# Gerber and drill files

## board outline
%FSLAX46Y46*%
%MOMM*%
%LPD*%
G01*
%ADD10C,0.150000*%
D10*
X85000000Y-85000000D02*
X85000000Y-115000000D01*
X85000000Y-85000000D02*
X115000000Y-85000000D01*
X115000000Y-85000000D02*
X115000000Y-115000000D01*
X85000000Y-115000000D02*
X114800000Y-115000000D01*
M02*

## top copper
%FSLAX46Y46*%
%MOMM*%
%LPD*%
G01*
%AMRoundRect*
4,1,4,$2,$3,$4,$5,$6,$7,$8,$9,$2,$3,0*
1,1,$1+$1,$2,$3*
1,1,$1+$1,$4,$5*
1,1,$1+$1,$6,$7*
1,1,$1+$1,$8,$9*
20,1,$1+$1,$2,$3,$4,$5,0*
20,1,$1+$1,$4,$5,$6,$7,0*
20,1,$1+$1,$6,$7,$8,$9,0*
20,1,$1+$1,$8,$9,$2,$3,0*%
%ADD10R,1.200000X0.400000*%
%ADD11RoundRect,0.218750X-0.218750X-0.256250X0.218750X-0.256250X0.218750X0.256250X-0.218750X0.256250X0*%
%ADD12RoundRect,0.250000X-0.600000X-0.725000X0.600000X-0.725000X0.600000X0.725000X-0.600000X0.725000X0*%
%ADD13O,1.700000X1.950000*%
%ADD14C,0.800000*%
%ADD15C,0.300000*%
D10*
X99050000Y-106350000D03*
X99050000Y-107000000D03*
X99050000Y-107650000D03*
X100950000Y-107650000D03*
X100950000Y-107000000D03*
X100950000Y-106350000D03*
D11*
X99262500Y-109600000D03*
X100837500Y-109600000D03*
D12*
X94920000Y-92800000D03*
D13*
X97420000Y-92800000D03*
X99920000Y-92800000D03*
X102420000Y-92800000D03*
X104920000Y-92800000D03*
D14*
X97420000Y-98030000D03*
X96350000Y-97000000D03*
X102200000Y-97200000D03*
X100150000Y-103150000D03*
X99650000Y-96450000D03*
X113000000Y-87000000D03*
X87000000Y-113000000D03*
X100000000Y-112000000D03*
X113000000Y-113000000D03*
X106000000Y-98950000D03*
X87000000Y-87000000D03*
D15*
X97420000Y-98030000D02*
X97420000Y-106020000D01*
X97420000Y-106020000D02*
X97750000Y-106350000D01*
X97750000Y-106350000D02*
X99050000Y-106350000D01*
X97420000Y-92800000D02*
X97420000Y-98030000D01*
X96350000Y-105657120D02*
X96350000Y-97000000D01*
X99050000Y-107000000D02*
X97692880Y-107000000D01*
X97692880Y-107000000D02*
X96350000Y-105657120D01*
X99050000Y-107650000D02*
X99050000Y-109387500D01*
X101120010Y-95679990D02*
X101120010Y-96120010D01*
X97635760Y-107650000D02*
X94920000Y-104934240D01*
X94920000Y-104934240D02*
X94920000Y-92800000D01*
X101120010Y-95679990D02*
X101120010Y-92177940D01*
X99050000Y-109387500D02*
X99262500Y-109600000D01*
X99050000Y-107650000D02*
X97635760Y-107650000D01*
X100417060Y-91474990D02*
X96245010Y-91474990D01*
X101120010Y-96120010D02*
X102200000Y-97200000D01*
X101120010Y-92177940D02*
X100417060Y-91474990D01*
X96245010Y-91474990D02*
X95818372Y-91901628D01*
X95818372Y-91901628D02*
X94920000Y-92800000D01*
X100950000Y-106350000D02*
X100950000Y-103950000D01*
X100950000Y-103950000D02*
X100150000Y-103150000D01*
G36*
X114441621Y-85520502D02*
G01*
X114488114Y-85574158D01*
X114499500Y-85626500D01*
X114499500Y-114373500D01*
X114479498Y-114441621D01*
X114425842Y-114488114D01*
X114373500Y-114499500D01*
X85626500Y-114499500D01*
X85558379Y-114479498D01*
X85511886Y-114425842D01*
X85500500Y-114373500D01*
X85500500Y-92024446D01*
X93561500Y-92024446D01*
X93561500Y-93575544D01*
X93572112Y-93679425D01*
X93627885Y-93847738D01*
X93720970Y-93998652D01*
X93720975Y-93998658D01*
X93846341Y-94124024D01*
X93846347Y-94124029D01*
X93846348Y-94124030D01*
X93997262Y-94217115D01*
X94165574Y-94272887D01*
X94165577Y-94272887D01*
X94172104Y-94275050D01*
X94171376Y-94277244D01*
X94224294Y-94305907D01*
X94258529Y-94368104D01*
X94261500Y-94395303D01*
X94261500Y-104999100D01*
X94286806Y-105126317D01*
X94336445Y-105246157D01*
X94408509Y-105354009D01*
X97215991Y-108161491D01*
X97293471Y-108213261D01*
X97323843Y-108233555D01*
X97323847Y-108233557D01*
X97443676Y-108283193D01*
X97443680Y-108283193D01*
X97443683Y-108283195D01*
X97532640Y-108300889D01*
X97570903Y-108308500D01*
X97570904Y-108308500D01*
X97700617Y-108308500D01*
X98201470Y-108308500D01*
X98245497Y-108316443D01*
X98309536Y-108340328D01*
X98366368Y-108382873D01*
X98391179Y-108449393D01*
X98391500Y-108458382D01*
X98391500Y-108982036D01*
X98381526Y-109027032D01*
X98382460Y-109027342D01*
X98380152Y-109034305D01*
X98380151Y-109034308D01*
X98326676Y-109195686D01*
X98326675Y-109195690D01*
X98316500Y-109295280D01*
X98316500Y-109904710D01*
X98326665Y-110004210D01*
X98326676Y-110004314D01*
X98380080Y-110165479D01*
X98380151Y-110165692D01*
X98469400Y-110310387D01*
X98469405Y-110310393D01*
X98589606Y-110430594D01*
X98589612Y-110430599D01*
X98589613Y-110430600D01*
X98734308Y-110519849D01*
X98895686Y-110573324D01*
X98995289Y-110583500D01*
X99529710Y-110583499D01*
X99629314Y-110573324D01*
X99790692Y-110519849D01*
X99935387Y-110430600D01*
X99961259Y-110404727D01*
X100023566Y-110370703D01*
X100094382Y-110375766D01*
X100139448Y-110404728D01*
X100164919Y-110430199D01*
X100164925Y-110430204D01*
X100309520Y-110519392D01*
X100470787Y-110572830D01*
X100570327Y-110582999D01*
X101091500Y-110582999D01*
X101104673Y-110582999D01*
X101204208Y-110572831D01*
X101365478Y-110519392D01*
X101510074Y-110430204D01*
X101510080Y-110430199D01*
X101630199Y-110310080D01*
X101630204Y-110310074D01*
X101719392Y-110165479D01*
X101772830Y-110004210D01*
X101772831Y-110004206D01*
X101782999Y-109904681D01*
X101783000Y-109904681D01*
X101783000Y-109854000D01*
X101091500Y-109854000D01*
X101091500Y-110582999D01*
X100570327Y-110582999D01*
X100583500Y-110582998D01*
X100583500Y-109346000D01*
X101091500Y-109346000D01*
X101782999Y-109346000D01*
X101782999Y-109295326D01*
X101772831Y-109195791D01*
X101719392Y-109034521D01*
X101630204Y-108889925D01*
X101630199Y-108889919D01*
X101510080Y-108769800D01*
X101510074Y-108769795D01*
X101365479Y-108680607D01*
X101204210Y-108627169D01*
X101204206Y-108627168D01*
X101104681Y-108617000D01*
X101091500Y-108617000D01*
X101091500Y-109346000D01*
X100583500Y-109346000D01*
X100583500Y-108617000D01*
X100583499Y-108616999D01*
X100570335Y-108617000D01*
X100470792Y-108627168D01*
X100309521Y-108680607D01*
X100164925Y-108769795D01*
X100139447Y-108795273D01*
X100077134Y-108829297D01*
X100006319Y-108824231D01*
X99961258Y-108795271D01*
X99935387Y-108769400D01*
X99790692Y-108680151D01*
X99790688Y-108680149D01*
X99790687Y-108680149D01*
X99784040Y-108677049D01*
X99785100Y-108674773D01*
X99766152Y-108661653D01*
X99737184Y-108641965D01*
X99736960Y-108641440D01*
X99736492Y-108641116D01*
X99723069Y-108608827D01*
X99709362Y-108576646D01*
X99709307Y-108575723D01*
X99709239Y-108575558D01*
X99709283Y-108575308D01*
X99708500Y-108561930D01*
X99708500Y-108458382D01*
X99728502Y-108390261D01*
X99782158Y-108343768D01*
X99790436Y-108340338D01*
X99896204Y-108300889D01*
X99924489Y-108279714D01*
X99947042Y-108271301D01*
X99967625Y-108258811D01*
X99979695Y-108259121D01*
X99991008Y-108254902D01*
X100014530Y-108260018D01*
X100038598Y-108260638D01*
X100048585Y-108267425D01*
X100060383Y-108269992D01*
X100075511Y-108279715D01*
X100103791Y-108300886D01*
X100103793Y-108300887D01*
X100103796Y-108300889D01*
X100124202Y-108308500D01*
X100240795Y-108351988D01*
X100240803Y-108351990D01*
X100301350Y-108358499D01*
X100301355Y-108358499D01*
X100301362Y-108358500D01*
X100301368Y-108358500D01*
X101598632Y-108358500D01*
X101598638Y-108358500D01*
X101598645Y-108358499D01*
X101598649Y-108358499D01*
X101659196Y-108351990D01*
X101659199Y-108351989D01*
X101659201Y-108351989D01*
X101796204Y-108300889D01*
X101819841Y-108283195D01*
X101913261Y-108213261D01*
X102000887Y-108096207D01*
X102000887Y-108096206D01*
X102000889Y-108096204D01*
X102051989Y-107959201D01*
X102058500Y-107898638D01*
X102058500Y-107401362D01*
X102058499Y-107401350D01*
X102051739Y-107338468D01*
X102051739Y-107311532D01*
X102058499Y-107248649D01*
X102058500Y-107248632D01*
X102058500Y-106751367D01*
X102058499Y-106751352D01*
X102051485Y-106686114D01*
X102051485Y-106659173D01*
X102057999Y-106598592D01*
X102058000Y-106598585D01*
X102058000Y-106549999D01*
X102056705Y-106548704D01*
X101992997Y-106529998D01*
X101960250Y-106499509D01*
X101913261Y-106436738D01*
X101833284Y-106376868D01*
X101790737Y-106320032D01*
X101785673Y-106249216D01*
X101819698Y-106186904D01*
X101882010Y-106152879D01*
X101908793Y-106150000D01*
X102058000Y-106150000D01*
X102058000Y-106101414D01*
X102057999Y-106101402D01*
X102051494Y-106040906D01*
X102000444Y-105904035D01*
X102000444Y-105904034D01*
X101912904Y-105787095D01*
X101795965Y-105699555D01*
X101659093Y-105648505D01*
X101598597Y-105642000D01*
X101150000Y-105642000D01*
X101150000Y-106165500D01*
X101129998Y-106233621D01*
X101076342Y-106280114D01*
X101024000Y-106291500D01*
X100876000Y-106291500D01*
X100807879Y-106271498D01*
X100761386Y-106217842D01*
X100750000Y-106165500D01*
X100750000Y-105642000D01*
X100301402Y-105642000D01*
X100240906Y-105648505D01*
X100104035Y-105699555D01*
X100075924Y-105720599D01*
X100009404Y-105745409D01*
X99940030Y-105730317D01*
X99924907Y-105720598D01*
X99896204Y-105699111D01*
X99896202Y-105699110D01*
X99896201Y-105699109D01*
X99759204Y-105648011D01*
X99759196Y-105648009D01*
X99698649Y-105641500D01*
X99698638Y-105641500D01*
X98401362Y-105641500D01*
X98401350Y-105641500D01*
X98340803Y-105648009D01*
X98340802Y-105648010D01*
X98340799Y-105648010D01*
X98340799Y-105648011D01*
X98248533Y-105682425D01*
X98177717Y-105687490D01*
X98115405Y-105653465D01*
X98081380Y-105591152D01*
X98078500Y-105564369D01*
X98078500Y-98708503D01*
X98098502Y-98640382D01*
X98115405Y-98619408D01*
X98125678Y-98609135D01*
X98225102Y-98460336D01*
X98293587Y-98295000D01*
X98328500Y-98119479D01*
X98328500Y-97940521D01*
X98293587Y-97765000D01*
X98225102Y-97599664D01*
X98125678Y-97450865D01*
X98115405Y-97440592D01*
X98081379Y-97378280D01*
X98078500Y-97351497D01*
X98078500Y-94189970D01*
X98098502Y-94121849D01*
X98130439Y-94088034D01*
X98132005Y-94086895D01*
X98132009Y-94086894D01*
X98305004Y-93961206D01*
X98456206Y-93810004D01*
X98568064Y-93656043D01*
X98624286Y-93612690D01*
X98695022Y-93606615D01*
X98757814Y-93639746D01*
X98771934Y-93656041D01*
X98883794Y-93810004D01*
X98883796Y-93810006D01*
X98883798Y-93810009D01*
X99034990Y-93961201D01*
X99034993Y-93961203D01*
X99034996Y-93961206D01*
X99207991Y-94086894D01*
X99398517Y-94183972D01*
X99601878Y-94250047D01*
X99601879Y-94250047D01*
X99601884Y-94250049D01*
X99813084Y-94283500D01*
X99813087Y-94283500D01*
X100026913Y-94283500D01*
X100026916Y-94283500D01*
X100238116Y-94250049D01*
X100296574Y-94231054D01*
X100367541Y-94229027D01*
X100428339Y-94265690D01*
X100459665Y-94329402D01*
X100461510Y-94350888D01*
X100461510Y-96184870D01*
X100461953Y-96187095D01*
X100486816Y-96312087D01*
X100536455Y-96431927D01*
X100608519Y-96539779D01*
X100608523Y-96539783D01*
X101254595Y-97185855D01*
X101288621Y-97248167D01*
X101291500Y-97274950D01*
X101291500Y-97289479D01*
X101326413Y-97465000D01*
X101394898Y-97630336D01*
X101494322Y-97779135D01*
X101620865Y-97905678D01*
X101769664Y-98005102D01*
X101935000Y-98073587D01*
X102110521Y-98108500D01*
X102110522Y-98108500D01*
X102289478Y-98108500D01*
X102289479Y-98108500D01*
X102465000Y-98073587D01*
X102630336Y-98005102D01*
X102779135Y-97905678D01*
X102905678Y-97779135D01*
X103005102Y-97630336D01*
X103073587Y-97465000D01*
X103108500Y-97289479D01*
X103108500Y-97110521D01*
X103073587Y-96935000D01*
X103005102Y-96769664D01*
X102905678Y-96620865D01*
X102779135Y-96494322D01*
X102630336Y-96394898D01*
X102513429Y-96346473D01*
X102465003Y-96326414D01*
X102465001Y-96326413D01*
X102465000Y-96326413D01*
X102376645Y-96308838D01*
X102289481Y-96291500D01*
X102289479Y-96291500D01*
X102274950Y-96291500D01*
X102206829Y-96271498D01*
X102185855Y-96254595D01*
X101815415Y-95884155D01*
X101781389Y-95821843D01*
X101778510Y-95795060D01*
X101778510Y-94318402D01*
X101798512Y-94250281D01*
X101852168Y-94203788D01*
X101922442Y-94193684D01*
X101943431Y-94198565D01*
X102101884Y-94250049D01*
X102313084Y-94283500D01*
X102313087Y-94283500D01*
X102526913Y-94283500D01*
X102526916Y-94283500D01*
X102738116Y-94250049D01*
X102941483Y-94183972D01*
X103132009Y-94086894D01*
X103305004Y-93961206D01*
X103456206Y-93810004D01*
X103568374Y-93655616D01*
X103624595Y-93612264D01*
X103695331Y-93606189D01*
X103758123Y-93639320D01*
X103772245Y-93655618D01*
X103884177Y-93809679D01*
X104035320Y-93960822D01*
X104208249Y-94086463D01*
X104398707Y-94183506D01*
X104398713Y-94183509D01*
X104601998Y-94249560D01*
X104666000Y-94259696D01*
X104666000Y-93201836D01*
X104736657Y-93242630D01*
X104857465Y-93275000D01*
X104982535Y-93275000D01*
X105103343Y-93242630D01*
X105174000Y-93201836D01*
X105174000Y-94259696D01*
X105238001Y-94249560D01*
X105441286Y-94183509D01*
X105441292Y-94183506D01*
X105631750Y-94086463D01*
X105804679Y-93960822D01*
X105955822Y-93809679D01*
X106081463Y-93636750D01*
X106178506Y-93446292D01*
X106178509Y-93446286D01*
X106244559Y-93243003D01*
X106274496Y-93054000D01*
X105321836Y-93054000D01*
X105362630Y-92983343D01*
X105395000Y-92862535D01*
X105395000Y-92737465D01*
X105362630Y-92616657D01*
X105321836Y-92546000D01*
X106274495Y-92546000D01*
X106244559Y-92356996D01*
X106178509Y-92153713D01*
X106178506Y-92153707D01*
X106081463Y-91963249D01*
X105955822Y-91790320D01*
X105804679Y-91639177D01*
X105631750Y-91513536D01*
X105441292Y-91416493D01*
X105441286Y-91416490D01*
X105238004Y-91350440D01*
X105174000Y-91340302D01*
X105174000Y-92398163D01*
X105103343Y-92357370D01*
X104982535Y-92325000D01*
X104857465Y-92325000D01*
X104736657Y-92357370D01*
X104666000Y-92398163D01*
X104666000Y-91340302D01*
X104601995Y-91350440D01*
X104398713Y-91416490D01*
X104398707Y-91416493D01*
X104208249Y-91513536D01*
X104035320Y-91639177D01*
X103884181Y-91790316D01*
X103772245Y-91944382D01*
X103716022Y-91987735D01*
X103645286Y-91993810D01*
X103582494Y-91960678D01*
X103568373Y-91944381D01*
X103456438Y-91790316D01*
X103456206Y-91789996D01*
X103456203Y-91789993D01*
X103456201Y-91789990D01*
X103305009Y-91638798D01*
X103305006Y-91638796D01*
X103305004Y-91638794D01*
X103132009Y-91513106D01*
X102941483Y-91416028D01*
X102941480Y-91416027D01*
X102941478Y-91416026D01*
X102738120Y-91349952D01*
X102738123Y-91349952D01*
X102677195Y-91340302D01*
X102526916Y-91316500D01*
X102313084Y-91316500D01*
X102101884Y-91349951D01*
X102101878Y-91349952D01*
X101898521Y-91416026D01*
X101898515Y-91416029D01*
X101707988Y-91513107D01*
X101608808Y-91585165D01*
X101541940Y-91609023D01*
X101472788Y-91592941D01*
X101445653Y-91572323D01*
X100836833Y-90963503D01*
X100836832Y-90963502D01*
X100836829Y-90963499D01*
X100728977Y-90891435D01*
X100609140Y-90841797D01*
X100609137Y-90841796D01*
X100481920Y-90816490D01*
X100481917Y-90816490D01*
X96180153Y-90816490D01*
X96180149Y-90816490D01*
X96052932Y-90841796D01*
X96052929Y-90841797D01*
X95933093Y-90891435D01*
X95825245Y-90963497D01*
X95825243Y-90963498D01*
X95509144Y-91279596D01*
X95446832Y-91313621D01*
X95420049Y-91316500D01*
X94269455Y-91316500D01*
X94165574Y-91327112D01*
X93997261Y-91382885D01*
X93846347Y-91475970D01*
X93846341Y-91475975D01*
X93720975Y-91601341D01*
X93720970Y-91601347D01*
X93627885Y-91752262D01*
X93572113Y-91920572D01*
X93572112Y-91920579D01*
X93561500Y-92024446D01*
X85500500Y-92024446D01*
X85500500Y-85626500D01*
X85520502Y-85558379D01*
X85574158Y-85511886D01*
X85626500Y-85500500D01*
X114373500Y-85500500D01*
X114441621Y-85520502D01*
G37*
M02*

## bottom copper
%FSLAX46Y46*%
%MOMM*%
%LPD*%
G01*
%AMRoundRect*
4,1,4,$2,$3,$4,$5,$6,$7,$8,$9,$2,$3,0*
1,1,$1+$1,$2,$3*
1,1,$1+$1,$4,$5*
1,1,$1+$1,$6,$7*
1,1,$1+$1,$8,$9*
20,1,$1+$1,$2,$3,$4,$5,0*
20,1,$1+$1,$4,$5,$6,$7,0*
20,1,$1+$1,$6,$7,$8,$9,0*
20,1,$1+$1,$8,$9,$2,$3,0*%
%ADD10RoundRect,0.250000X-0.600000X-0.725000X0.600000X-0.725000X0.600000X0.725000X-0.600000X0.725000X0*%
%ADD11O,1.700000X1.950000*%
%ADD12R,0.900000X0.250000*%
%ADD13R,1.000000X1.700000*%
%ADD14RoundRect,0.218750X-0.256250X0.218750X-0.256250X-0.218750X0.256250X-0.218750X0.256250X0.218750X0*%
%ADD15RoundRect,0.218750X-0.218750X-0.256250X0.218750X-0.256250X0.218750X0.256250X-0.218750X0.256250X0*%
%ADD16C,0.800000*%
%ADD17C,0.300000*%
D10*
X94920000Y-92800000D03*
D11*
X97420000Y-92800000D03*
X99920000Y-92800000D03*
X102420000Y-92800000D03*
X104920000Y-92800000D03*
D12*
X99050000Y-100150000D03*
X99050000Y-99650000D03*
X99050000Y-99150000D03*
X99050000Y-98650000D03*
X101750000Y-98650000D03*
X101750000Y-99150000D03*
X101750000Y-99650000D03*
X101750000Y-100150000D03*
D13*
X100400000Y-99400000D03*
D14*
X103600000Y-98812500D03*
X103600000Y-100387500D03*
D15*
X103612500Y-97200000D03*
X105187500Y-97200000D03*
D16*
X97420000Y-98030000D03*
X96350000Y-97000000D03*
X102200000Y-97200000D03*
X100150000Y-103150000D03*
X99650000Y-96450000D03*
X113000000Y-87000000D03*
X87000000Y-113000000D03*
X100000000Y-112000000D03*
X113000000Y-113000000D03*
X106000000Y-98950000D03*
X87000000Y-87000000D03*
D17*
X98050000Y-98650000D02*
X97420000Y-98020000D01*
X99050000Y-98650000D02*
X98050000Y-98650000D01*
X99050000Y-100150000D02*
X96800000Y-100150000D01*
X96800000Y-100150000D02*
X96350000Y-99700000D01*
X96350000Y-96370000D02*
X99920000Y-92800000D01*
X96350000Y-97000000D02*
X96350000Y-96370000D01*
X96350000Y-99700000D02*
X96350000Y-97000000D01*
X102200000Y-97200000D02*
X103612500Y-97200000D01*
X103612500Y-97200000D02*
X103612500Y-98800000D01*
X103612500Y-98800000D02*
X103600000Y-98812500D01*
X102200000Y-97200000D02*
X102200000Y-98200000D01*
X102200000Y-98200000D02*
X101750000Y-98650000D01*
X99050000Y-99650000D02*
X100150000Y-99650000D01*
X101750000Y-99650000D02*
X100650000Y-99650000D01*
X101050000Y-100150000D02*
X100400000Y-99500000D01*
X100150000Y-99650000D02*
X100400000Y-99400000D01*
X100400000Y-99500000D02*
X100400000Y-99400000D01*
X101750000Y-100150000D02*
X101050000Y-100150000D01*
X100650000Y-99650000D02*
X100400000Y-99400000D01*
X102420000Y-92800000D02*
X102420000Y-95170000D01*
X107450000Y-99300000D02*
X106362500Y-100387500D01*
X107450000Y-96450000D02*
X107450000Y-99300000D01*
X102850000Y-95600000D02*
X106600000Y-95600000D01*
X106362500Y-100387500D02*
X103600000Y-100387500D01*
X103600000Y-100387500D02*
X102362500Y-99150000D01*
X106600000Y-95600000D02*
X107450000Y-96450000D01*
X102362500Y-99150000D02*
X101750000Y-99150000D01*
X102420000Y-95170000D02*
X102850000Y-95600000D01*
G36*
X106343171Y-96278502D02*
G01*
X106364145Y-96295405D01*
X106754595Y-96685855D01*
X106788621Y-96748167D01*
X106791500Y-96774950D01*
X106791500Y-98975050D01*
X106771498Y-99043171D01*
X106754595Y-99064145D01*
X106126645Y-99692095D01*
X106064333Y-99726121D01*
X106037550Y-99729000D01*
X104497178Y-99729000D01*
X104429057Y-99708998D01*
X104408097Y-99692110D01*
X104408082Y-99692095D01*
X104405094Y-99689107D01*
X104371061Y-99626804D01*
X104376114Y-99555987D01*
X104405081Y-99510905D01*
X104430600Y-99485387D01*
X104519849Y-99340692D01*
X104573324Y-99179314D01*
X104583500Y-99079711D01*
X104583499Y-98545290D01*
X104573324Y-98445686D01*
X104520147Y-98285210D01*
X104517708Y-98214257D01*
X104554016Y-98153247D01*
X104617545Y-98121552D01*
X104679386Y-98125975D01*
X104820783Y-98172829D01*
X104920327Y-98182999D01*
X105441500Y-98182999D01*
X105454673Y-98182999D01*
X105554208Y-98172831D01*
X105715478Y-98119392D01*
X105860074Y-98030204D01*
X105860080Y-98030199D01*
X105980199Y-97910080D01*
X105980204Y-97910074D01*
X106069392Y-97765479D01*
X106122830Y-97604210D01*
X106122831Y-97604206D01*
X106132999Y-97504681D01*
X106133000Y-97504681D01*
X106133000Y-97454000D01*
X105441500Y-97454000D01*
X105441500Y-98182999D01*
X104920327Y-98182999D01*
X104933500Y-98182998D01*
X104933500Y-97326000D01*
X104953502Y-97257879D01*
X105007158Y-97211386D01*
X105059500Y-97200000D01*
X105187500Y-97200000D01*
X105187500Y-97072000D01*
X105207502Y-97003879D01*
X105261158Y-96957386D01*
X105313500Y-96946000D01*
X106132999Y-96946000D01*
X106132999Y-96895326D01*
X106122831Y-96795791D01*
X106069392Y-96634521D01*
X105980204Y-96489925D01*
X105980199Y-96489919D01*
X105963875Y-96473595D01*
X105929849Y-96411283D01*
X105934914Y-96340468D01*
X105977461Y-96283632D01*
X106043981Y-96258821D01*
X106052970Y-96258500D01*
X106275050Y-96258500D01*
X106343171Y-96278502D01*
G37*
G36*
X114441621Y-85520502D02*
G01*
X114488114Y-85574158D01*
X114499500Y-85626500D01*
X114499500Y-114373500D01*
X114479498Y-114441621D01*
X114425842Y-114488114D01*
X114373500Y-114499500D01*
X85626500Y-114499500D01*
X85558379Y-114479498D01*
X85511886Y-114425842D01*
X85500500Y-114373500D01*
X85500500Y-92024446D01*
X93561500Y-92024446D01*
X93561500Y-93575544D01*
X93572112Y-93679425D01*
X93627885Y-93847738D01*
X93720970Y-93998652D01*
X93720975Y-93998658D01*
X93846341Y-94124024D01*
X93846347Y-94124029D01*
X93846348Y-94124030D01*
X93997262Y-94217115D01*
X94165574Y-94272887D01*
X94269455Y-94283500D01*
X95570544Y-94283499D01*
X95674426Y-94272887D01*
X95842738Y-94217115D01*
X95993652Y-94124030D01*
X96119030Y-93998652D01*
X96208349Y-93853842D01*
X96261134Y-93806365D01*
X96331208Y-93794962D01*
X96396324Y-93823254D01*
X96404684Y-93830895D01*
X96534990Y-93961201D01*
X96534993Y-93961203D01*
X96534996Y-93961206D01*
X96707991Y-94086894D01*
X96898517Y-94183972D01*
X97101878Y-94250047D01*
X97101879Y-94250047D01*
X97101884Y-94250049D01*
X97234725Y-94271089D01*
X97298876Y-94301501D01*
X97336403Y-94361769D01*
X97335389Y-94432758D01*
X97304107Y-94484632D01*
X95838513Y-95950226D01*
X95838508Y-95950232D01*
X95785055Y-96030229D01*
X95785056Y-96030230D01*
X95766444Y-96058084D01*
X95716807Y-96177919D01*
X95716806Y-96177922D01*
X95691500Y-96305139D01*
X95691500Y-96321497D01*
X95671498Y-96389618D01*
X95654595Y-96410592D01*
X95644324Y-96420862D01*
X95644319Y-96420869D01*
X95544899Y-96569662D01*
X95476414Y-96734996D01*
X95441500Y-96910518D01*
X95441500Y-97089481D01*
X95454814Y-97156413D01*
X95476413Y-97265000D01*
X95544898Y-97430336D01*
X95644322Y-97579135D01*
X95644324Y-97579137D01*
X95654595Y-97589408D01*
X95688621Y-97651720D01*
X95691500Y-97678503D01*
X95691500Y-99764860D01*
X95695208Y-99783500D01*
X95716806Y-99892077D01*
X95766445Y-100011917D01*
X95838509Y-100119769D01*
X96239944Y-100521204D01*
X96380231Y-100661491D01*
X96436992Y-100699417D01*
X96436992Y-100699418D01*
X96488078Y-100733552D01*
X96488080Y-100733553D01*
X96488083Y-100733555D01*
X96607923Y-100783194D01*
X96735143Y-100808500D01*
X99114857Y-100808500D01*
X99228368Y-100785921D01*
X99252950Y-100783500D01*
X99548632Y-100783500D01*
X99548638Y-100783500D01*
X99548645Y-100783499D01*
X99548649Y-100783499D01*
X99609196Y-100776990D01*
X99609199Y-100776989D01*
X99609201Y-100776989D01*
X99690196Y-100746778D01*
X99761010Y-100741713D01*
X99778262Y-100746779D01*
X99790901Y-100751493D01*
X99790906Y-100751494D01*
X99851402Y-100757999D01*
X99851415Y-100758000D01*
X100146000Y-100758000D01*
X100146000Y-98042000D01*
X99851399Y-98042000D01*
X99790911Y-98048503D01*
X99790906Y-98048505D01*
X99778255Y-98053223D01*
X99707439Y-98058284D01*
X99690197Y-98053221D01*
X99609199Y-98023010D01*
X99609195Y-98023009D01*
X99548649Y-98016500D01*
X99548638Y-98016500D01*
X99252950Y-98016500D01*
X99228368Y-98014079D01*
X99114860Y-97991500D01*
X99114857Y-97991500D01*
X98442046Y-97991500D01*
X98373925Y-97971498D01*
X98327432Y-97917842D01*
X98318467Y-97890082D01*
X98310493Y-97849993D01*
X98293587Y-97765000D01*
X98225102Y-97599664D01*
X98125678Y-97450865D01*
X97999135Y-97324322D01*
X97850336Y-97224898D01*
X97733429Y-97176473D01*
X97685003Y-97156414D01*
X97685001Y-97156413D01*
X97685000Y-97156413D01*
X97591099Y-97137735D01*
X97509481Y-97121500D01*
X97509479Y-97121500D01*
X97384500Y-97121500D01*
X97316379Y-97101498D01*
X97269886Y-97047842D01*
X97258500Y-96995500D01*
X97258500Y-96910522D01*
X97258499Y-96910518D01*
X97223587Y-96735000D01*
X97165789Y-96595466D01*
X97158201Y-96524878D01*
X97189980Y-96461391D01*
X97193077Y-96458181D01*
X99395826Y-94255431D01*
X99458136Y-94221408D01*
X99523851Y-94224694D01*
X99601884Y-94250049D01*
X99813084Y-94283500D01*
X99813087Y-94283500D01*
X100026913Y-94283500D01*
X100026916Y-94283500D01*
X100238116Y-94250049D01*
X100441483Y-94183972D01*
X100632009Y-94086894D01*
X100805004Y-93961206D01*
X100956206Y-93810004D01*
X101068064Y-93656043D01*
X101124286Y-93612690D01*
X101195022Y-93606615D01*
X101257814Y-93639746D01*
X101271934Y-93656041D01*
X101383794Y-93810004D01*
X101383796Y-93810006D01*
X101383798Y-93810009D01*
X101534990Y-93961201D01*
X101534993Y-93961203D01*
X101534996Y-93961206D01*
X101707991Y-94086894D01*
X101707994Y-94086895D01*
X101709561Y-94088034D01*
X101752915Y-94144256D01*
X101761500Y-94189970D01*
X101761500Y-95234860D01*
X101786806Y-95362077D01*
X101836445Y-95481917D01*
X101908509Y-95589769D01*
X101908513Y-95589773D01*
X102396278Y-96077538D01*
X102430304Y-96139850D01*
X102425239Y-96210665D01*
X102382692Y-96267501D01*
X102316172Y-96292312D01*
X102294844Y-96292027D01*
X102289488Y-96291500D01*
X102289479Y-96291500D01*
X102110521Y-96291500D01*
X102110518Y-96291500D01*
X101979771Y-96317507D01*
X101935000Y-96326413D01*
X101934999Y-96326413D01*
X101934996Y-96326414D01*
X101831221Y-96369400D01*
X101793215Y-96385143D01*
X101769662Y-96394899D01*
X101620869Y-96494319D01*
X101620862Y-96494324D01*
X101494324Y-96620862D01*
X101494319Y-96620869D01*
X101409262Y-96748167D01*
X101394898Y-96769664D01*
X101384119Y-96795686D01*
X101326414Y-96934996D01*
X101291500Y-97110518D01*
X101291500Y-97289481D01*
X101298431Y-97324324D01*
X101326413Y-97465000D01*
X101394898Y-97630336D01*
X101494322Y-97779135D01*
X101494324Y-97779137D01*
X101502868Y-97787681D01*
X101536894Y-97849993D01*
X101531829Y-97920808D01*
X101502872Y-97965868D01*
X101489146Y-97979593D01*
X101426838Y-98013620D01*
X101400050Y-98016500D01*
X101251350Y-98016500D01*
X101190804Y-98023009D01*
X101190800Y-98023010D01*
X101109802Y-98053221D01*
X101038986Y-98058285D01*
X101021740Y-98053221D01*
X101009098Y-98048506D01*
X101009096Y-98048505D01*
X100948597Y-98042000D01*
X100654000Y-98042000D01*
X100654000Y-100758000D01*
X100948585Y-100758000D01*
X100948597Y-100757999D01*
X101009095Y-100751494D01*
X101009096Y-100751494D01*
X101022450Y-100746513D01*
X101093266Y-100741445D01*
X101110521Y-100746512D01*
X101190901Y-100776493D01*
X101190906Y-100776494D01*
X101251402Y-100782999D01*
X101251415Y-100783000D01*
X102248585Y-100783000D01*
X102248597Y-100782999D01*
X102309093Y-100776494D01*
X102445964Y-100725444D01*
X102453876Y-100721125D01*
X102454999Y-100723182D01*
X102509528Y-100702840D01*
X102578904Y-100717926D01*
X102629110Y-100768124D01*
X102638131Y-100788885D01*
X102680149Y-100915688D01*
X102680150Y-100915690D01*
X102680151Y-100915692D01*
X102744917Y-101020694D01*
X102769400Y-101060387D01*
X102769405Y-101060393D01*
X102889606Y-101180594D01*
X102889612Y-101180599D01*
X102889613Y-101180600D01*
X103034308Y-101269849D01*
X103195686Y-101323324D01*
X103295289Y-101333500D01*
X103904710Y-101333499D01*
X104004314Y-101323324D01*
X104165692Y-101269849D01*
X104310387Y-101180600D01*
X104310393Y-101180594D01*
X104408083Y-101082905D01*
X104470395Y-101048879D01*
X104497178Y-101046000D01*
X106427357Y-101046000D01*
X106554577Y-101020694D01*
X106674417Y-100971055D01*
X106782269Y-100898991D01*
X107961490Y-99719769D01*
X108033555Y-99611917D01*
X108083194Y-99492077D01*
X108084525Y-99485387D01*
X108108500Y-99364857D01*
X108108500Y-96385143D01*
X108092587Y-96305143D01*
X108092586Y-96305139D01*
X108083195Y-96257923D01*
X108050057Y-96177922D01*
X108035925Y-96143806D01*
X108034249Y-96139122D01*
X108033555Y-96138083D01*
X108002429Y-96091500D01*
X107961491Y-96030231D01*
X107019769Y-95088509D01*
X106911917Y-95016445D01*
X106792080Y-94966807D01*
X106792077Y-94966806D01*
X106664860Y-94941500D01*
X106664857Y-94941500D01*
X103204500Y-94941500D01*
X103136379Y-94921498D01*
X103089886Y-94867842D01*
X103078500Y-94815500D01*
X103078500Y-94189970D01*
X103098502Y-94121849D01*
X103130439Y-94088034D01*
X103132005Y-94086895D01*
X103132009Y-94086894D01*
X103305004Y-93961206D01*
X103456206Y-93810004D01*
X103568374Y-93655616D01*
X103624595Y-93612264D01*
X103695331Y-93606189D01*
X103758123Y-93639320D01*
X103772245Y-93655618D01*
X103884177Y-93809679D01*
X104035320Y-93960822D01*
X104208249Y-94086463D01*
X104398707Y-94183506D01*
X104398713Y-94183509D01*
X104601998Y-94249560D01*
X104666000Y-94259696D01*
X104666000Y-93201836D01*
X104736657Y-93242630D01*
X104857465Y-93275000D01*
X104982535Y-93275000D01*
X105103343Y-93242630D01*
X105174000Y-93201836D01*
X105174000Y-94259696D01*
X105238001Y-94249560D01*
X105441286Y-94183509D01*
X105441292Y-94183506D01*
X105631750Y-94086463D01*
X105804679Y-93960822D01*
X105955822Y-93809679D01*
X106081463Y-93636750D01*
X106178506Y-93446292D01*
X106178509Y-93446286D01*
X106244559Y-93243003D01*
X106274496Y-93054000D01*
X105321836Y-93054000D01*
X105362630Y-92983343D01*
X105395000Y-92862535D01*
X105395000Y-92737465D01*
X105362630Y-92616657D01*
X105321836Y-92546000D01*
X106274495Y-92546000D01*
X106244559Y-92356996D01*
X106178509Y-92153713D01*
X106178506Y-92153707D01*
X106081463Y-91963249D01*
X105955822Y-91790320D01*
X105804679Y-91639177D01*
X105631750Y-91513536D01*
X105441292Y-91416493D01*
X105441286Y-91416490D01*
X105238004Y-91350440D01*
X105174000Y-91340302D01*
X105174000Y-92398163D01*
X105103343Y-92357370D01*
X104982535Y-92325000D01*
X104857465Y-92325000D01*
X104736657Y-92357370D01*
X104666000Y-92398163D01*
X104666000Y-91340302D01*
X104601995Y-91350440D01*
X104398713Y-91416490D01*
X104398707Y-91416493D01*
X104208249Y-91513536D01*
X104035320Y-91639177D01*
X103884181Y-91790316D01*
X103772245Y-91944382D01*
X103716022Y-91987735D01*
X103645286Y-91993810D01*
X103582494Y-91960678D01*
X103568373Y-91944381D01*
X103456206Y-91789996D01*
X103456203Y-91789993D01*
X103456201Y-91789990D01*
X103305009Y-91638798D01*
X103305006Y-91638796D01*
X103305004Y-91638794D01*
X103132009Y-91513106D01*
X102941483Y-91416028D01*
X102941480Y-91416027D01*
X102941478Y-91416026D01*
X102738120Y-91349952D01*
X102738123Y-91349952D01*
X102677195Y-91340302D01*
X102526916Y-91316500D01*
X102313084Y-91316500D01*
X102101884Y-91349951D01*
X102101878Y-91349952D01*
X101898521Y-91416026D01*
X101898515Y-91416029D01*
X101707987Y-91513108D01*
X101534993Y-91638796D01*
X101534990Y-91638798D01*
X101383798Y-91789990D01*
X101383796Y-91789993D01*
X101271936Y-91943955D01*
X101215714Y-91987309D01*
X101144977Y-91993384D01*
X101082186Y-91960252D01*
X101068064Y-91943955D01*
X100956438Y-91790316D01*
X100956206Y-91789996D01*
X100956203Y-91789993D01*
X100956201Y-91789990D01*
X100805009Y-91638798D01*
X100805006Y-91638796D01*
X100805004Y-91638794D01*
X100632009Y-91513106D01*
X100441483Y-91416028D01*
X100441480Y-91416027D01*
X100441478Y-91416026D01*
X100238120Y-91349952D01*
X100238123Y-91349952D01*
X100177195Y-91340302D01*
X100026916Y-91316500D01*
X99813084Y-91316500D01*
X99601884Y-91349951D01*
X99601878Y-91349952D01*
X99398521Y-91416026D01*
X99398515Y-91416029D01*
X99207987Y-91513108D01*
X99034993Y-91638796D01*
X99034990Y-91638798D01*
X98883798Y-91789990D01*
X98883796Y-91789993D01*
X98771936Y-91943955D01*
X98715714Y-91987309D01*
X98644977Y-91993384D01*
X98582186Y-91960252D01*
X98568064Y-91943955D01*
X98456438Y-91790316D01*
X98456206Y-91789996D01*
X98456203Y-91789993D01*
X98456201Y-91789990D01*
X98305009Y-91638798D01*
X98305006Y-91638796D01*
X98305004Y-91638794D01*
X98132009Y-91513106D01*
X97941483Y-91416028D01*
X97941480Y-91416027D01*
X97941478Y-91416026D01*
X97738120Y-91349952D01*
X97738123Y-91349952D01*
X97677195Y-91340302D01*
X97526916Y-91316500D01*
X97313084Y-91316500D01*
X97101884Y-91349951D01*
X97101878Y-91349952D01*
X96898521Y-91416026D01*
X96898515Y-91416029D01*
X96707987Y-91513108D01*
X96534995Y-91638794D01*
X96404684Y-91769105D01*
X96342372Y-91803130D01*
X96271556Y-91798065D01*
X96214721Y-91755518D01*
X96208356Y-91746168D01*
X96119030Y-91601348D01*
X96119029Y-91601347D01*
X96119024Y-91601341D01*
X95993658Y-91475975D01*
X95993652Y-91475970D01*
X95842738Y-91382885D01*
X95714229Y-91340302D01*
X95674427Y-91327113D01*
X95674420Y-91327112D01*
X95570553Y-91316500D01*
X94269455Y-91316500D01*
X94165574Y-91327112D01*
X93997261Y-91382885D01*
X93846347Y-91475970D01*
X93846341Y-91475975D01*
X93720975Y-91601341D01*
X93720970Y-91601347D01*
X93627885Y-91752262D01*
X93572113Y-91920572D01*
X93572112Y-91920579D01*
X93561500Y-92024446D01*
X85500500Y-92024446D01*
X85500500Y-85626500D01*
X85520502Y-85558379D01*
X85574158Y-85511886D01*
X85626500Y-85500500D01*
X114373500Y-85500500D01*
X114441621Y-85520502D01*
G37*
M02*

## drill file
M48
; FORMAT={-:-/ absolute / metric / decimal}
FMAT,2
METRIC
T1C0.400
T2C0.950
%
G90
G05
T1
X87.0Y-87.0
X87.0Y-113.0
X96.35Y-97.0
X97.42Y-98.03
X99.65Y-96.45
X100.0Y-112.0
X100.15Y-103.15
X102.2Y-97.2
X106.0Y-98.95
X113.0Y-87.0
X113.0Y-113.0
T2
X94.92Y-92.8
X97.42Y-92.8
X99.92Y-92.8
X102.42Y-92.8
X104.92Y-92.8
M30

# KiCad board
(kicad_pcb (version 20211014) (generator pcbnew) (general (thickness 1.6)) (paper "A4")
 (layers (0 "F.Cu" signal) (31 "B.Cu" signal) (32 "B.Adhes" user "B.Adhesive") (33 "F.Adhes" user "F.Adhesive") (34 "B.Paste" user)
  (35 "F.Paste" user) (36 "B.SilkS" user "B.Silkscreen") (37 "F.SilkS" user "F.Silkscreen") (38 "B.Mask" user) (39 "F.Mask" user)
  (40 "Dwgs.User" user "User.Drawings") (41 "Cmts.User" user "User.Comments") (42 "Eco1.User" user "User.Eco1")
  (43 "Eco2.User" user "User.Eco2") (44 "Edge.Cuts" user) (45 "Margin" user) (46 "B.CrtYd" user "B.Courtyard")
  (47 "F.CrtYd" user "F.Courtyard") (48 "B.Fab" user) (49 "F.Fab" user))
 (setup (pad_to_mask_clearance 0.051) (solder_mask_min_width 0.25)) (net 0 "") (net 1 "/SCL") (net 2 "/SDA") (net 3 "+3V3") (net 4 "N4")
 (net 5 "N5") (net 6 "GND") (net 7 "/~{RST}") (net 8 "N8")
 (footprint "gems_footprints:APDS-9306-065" (layer "F.Cu") (at 100 107 90)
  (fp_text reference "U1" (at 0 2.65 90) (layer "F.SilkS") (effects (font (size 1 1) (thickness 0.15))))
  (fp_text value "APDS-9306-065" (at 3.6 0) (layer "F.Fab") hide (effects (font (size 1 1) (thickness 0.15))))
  (pad "1" smd rect locked (at 0.65 -0.95 90) (size 0.4 1.2) (layers "F.Cu" "F.Paste" "F.Mask") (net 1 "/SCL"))
  (pad "2" smd rect locked (at 0 -0.95 90) (size 0.4 1.2) (layers "F.Cu" "F.Paste" "F.Mask") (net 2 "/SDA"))
  (pad "3" smd rect locked (at -0.65 -0.95 90) (size 0.4 1.2) (layers "F.Cu" "F.Paste" "F.Mask") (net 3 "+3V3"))
  (pad "4" smd rect locked (at -0.65 0.95 90) (size 0.4 1.2) (layers "F.Cu" "F.Paste" "F.Mask") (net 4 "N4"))
  (pad "5" smd rect locked (at 0 0.95 90) (size 0.4 1.2) (layers "F.Cu" "F.Paste" "F.Mask") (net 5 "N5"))
  (pad "6" smd rect locked (at 0.65 0.95 90) (size 0.4 1.2) (layers "F.Cu" "F.Paste" "F.Mask") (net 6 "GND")))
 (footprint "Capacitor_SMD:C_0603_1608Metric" (layer "F.Cu") (at 100.05 109.6)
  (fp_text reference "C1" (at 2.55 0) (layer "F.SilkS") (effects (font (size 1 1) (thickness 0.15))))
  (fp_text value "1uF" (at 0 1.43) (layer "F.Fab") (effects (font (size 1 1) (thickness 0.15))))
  (pad "1" smd roundrect locked (at -0.7875 0) (size 0.875 0.95) (layers "F.Cu" "F.Paste" "F.Mask") (roundrect_rratio 0.25) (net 3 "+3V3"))
  (pad "2" smd roundrect locked (at 0.7875 0) (size 0.875 0.95) (layers "F.Cu" "F.Paste" "F.Mask") (roundrect_rratio 0.25) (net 6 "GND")))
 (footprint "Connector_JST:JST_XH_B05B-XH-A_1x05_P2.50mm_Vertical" (layer "B.Cu") (at 94.92 92.8)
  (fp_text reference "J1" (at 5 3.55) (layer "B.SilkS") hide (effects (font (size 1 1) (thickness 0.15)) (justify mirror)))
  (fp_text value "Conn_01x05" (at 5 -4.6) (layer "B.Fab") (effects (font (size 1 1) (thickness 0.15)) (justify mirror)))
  (pad "1" thru_hole roundrect locked (at 0 0) (size 1.7 1.95) (drill 0.95) (layers *.Cu *.Mask) (roundrect_rratio 0.147059) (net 3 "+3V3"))
  (pad "2" thru_hole oval locked (at 2.5 0) (size 1.7 1.95) (drill 0.95) (layers *.Cu *.Mask) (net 1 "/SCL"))
  (pad "3" thru_hole oval locked (at 5 0) (size 1.7 1.95) (drill 0.95) (layers *.Cu *.Mask) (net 2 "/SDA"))
  (pad "4" thru_hole oval locked (at 7.5 0) (size 1.7 1.95) (drill 0.95) (layers *.Cu *.Mask) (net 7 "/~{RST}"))
  (pad "5" thru_hole oval locked (at 10 0) (size 1.7 1.95) (drill 0.95) (layers *.Cu *.Mask) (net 6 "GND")))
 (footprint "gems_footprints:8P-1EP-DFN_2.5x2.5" (layer "B.Cu") (at 100.4 99.4)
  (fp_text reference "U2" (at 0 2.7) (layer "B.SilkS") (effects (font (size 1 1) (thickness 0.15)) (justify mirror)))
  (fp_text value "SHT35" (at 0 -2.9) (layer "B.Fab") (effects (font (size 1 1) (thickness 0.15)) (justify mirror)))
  (pad "1" smd rect locked (at -1.35 0.75) (size 0.9 0.25) (layers "B.Cu" "B.Paste" "B.Mask") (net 2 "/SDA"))
  (pad "2" smd rect locked (at -1.35 0.25) (size 0.9 0.25) (layers "B.Cu" "B.Paste" "B.Mask") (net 6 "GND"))
  (pad "3" smd rect locked (at -1.35 -0.25) (size 0.9 0.25) (layers "B.Cu" "B.Paste" "B.Mask") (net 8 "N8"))
  (pad "4" smd rect locked (at -1.35 -0.75) (size 0.9 0.25) (layers "B.Cu" "B.Paste" "B.Mask") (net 1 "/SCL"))
  (pad "5" smd rect locked (at 1.35 -0.75) (size 0.9 0.25) (layers "B.Cu" "B.Paste" "B.Mask") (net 3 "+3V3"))
  (pad "6" smd rect locked (at 1.35 -0.25) (size 0.9 0.25) (layers "B.Cu" "B.Paste" "B.Mask") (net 7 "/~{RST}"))
  (pad "7" smd rect locked (at 1.35 0.25) (size 0.9 0.25) (layers "B.Cu" "B.Paste" "B.Mask") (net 6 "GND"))
  (pad "8" smd rect locked (at 1.35 0.75) (size 0.9 0.25) (layers "B.Cu" "B.Paste" "B.Mask") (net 6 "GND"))
  (pad "9" smd rect locked (at 0 0) (size 1 1.7) (layers "B.Cu" "B.Mask") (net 6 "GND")))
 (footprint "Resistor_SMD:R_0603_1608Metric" (layer "B.Cu") (at 103.6 99.6 -90)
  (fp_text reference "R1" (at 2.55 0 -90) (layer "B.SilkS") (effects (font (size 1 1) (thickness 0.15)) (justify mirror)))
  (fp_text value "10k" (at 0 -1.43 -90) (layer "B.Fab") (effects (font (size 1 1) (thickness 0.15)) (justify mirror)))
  (pad "1" smd roundrect locked (at -0.7875 0 270) (size 0.875 0.95) (layers "B.Cu" "B.Paste" "B.Mask") (roundrect_rratio 0.25)
   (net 3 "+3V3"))
  (pad "2" smd roundrect locked (at 0.7875 0 270) (size 0.875 0.95) (layers "B.Cu" "B.Paste" "B.Mask") (roundrect_rratio 0.25)
   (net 7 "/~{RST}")))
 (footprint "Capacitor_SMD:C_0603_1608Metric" (layer "B.Cu") (at 104.4 97.2)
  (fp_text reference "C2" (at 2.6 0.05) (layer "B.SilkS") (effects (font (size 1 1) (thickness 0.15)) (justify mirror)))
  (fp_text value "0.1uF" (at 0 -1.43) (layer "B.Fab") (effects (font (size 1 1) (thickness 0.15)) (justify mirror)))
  (pad "1" smd roundrect locked (at -0.7875 0) (size 0.875 0.95) (layers "B.Cu" "B.Paste" "B.Mask") (roundrect_rratio 0.25) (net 3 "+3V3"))
  (pad "2" smd roundrect locked (at 0.7875 0) (size 0.875 0.95) (layers "B.Cu" "B.Paste" "B.Mask") (roundrect_rratio 0.25) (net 6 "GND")))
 (gr_line (start 85 85) (end 85 115) (layer "Edge.Cuts") (width 0.15))
 (gr_line (start 85 85) (end 115 85) (layer "Edge.Cuts") (width 0.15))
 (gr_line (start 115 85) (end 115 115) (layer "Edge.Cuts") (width 0.15))
 (gr_line (start 85 115) (end 114.8 115) (layer "Edge.Cuts") (width 0.15))
 (segment (start 97.42 98.03) (end 97.42 106.02) (width 0.3) (layer "F.Cu") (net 1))
 (segment (start 97.42 106.02) (end 97.75 106.35) (width 0.3) (layer "F.Cu") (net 1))
 (segment (start 97.75 106.35) (end 99.05 106.35) (width 0.3) (layer "F.Cu") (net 1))
 (segment (start 97.42 92.8) (end 97.42 98.03) (width 0.3) (layer "F.Cu") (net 1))
 (via (at 97.42 98.03) (size 0.8) (drill 0.4) (layers "F.Cu" "B.Cu") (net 1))
 (segment (start 98.05 98.65) (end 97.42 98.02) (width 0.3) (layer "B.Cu") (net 1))
 (segment (start 99.05 98.65) (end 98.05 98.65) (width 0.3) (layer "B.Cu") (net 1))
 (segment (start 96.35 105.65712) (end 96.35 97) (width 0.3) (layer "F.Cu") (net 2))
 (segment (start 99.05 107) (end 97.69288 107) (width 0.3) (layer "F.Cu") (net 2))
 (segment (start 97.69288 107) (end 96.35 105.65712) (width 0.3) (layer "F.Cu") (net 2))
 (via (at 96.35 97) (size 0.8) (drill 0.4) (layers "F.Cu" "B.Cu") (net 2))
 (segment (start 99.05 100.15) (end 96.8 100.15) (width 0.3) (layer "B.Cu") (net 2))
 (segment (start 96.8 100.15) (end 96.35 99.7) (width 0.3) (layer "B.Cu") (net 2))
 (segment (start 96.35 96.37) (end 99.92 92.8) (width 0.3) (layer "B.Cu") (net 2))
 (segment (start 96.35 97) (end 96.35 96.37) (width 0.3) (layer "B.Cu") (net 2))
 (segment (start 96.35 99.7) (end 96.35 97) (width 0.3) (layer "B.Cu") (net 2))
 (segment (start 99.05 107.65) (end 99.05 109.3875) (width 0.3) (layer "F.Cu") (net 3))
 (segment (start 101.12001 95.67999) (end 101.12001 96.12001) (width 0.3) (layer "F.Cu") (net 3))
 (segment (start 97.63576 107.65) (end 94.92 104.93424) (width 0.3) (layer "F.Cu") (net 3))
 (segment (start 94.92 104.93424) (end 94.92 92.8) (width 0.3) (layer "F.Cu") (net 3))
 (segment (start 101.12001 95.67999) (end 101.12001 92.17794) (width 0.3) (layer "F.Cu") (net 3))
 (segment (start 99.05 109.3875) (end 99.2625 109.6) (width 0.3) (layer "F.Cu") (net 3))
 (segment (start 99.05 107.65) (end 97.63576 107.65) (width 0.3) (layer "F.Cu") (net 3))
 (segment (start 100.41706 91.47499) (end 96.24501 91.47499) (width 0.3) (layer "F.Cu") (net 3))
 (segment (start 101.12001 96.12001) (end 102.2 97.2) (width 0.3) (layer "F.Cu") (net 3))
 (segment (start 101.12001 92.17794) (end 100.41706 91.47499) (width 0.3) (layer "F.Cu") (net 3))
 (segment (start 96.24501 91.47499) (end 95.818372 91.901628) (width 0.3) (layer "F.Cu") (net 3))
 (segment (start 95.818372 91.901628) (end 94.92 92.8) (width 0.3) (layer "F.Cu") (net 3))
 (via (at 102.2 97.2) (size 0.8) (drill 0.4) (layers "F.Cu" "B.Cu") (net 3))
 (segment (start 102.2 97.2) (end 103.6125 97.2) (width 0.3) (layer "B.Cu") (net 3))
 (segment (start 103.6125 97.2) (end 103.6125 98.8) (width 0.3) (layer "B.Cu") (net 3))
 (segment (start 103.6125 98.8) (end 103.6 98.8125) (width 0.3) (layer "B.Cu") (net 3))
 (segment (start 102.2 97.2) (end 102.2 98.2) (width 0.3) (layer "B.Cu") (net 3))
 (segment (start 102.2 98.2) (end 101.75 98.65) (width 0.3) (layer "B.Cu") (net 3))
 (segment (start 100.95 106.35) (end 100.95 103.95) (width 0.3) (layer "F.Cu") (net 6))
 (segment (start 100.95 103.95) (end 100.15 103.15) (width 0.3) (layer "F.Cu") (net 6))
 (via (at 100.15 103.15) (size 0.8) (drill 0.4) (layers "F.Cu" "B.Cu") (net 6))
 (via (at 99.65 96.45) (size 0.8) (drill 0.4) (layers "F.Cu" "B.Cu") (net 6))
 (via (at 113 87) (size 0.8) (drill 0.4) (layers "F.Cu" "B.Cu") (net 6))
 (via (at 87 113) (size 0.8) (drill 0.4) (layers "F.Cu" "B.Cu") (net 6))
 (via (at 100 112) (size 0.8) (drill 0.4) (layers "F.Cu" "B.Cu") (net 6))
 (via (at 113 113) (size 0.8) (drill 0.4) (layers "F.Cu" "B.Cu") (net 6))
 (via (at 106 98.95) (size 0.8) (drill 0.4) (layers "F.Cu" "B.Cu") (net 6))
 (via (at 87 87) (size 0.8) (drill 0.4) (layers "F.Cu" "B.Cu") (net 6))
 (segment (start 99.05 99.65) (end 100.15 99.65) (width 0.3) (layer "B.Cu") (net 6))
 (segment (start 101.75 99.65) (end 100.65 99.65) (width 0.3) (layer "B.Cu") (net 6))
 (segment (start 101.05 100.15) (end 100.4 99.5) (width 0.3) (layer "B.Cu") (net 6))
 (segment (start 100.15 99.65) (end 100.4 99.4) (width 0.3) (layer "B.Cu") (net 6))
 (segment (start 100.4 99.5) (end 100.4 99.4) (width 0.3) (layer "B.Cu") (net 6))
 (segment (start 101.75 100.15) (end 101.05 100.15) (width 0.3) (layer "B.Cu") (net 6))
 (segment (start 100.65 99.65) (end 100.4 99.4) (width 0.3) (layer "B.Cu") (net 6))
 (segment (start 102.42 92.8) (end 102.42 95.17) (width 0.3) (layer "B.Cu") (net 7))
 (segment (start 107.45 99.3) (end 106.3625 100.3875) (width 0.3) (layer "B.Cu") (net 7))
 (segment (start 107.45 96.45) (end 107.45 99.3) (width 0.3) (layer "B.Cu") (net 7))
 (segment (start 102.85 95.6) (end 106.6 95.6) (width 0.3) (layer "B.Cu") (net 7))
 (segment (start 106.3625 100.3875) (end 103.6 100.3875) (width 0.3) (layer "B.Cu") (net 7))
 (segment (start 103.6 100.3875) (end 102.3625 99.15) (width 0.3) (layer "B.Cu") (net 7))
 (segment (start 106.6 95.6) (end 107.45 96.45) (width 0.3) (layer "B.Cu") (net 7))
 (segment (start 102.3625 99.15) (end 101.75 99.15) (width 0.3) (layer "B.Cu") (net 7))
 (segment (start 102.42 95.17) (end 102.85 95.6) (width 0.3) (layer "B.Cu") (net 7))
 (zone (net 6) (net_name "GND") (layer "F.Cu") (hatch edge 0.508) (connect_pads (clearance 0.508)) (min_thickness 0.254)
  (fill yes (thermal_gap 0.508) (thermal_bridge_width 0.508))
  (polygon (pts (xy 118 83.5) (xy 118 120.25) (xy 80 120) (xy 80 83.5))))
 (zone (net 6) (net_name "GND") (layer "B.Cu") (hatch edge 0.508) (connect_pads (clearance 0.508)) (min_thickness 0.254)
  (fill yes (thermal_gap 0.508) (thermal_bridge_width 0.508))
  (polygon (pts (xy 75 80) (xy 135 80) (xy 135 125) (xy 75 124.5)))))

